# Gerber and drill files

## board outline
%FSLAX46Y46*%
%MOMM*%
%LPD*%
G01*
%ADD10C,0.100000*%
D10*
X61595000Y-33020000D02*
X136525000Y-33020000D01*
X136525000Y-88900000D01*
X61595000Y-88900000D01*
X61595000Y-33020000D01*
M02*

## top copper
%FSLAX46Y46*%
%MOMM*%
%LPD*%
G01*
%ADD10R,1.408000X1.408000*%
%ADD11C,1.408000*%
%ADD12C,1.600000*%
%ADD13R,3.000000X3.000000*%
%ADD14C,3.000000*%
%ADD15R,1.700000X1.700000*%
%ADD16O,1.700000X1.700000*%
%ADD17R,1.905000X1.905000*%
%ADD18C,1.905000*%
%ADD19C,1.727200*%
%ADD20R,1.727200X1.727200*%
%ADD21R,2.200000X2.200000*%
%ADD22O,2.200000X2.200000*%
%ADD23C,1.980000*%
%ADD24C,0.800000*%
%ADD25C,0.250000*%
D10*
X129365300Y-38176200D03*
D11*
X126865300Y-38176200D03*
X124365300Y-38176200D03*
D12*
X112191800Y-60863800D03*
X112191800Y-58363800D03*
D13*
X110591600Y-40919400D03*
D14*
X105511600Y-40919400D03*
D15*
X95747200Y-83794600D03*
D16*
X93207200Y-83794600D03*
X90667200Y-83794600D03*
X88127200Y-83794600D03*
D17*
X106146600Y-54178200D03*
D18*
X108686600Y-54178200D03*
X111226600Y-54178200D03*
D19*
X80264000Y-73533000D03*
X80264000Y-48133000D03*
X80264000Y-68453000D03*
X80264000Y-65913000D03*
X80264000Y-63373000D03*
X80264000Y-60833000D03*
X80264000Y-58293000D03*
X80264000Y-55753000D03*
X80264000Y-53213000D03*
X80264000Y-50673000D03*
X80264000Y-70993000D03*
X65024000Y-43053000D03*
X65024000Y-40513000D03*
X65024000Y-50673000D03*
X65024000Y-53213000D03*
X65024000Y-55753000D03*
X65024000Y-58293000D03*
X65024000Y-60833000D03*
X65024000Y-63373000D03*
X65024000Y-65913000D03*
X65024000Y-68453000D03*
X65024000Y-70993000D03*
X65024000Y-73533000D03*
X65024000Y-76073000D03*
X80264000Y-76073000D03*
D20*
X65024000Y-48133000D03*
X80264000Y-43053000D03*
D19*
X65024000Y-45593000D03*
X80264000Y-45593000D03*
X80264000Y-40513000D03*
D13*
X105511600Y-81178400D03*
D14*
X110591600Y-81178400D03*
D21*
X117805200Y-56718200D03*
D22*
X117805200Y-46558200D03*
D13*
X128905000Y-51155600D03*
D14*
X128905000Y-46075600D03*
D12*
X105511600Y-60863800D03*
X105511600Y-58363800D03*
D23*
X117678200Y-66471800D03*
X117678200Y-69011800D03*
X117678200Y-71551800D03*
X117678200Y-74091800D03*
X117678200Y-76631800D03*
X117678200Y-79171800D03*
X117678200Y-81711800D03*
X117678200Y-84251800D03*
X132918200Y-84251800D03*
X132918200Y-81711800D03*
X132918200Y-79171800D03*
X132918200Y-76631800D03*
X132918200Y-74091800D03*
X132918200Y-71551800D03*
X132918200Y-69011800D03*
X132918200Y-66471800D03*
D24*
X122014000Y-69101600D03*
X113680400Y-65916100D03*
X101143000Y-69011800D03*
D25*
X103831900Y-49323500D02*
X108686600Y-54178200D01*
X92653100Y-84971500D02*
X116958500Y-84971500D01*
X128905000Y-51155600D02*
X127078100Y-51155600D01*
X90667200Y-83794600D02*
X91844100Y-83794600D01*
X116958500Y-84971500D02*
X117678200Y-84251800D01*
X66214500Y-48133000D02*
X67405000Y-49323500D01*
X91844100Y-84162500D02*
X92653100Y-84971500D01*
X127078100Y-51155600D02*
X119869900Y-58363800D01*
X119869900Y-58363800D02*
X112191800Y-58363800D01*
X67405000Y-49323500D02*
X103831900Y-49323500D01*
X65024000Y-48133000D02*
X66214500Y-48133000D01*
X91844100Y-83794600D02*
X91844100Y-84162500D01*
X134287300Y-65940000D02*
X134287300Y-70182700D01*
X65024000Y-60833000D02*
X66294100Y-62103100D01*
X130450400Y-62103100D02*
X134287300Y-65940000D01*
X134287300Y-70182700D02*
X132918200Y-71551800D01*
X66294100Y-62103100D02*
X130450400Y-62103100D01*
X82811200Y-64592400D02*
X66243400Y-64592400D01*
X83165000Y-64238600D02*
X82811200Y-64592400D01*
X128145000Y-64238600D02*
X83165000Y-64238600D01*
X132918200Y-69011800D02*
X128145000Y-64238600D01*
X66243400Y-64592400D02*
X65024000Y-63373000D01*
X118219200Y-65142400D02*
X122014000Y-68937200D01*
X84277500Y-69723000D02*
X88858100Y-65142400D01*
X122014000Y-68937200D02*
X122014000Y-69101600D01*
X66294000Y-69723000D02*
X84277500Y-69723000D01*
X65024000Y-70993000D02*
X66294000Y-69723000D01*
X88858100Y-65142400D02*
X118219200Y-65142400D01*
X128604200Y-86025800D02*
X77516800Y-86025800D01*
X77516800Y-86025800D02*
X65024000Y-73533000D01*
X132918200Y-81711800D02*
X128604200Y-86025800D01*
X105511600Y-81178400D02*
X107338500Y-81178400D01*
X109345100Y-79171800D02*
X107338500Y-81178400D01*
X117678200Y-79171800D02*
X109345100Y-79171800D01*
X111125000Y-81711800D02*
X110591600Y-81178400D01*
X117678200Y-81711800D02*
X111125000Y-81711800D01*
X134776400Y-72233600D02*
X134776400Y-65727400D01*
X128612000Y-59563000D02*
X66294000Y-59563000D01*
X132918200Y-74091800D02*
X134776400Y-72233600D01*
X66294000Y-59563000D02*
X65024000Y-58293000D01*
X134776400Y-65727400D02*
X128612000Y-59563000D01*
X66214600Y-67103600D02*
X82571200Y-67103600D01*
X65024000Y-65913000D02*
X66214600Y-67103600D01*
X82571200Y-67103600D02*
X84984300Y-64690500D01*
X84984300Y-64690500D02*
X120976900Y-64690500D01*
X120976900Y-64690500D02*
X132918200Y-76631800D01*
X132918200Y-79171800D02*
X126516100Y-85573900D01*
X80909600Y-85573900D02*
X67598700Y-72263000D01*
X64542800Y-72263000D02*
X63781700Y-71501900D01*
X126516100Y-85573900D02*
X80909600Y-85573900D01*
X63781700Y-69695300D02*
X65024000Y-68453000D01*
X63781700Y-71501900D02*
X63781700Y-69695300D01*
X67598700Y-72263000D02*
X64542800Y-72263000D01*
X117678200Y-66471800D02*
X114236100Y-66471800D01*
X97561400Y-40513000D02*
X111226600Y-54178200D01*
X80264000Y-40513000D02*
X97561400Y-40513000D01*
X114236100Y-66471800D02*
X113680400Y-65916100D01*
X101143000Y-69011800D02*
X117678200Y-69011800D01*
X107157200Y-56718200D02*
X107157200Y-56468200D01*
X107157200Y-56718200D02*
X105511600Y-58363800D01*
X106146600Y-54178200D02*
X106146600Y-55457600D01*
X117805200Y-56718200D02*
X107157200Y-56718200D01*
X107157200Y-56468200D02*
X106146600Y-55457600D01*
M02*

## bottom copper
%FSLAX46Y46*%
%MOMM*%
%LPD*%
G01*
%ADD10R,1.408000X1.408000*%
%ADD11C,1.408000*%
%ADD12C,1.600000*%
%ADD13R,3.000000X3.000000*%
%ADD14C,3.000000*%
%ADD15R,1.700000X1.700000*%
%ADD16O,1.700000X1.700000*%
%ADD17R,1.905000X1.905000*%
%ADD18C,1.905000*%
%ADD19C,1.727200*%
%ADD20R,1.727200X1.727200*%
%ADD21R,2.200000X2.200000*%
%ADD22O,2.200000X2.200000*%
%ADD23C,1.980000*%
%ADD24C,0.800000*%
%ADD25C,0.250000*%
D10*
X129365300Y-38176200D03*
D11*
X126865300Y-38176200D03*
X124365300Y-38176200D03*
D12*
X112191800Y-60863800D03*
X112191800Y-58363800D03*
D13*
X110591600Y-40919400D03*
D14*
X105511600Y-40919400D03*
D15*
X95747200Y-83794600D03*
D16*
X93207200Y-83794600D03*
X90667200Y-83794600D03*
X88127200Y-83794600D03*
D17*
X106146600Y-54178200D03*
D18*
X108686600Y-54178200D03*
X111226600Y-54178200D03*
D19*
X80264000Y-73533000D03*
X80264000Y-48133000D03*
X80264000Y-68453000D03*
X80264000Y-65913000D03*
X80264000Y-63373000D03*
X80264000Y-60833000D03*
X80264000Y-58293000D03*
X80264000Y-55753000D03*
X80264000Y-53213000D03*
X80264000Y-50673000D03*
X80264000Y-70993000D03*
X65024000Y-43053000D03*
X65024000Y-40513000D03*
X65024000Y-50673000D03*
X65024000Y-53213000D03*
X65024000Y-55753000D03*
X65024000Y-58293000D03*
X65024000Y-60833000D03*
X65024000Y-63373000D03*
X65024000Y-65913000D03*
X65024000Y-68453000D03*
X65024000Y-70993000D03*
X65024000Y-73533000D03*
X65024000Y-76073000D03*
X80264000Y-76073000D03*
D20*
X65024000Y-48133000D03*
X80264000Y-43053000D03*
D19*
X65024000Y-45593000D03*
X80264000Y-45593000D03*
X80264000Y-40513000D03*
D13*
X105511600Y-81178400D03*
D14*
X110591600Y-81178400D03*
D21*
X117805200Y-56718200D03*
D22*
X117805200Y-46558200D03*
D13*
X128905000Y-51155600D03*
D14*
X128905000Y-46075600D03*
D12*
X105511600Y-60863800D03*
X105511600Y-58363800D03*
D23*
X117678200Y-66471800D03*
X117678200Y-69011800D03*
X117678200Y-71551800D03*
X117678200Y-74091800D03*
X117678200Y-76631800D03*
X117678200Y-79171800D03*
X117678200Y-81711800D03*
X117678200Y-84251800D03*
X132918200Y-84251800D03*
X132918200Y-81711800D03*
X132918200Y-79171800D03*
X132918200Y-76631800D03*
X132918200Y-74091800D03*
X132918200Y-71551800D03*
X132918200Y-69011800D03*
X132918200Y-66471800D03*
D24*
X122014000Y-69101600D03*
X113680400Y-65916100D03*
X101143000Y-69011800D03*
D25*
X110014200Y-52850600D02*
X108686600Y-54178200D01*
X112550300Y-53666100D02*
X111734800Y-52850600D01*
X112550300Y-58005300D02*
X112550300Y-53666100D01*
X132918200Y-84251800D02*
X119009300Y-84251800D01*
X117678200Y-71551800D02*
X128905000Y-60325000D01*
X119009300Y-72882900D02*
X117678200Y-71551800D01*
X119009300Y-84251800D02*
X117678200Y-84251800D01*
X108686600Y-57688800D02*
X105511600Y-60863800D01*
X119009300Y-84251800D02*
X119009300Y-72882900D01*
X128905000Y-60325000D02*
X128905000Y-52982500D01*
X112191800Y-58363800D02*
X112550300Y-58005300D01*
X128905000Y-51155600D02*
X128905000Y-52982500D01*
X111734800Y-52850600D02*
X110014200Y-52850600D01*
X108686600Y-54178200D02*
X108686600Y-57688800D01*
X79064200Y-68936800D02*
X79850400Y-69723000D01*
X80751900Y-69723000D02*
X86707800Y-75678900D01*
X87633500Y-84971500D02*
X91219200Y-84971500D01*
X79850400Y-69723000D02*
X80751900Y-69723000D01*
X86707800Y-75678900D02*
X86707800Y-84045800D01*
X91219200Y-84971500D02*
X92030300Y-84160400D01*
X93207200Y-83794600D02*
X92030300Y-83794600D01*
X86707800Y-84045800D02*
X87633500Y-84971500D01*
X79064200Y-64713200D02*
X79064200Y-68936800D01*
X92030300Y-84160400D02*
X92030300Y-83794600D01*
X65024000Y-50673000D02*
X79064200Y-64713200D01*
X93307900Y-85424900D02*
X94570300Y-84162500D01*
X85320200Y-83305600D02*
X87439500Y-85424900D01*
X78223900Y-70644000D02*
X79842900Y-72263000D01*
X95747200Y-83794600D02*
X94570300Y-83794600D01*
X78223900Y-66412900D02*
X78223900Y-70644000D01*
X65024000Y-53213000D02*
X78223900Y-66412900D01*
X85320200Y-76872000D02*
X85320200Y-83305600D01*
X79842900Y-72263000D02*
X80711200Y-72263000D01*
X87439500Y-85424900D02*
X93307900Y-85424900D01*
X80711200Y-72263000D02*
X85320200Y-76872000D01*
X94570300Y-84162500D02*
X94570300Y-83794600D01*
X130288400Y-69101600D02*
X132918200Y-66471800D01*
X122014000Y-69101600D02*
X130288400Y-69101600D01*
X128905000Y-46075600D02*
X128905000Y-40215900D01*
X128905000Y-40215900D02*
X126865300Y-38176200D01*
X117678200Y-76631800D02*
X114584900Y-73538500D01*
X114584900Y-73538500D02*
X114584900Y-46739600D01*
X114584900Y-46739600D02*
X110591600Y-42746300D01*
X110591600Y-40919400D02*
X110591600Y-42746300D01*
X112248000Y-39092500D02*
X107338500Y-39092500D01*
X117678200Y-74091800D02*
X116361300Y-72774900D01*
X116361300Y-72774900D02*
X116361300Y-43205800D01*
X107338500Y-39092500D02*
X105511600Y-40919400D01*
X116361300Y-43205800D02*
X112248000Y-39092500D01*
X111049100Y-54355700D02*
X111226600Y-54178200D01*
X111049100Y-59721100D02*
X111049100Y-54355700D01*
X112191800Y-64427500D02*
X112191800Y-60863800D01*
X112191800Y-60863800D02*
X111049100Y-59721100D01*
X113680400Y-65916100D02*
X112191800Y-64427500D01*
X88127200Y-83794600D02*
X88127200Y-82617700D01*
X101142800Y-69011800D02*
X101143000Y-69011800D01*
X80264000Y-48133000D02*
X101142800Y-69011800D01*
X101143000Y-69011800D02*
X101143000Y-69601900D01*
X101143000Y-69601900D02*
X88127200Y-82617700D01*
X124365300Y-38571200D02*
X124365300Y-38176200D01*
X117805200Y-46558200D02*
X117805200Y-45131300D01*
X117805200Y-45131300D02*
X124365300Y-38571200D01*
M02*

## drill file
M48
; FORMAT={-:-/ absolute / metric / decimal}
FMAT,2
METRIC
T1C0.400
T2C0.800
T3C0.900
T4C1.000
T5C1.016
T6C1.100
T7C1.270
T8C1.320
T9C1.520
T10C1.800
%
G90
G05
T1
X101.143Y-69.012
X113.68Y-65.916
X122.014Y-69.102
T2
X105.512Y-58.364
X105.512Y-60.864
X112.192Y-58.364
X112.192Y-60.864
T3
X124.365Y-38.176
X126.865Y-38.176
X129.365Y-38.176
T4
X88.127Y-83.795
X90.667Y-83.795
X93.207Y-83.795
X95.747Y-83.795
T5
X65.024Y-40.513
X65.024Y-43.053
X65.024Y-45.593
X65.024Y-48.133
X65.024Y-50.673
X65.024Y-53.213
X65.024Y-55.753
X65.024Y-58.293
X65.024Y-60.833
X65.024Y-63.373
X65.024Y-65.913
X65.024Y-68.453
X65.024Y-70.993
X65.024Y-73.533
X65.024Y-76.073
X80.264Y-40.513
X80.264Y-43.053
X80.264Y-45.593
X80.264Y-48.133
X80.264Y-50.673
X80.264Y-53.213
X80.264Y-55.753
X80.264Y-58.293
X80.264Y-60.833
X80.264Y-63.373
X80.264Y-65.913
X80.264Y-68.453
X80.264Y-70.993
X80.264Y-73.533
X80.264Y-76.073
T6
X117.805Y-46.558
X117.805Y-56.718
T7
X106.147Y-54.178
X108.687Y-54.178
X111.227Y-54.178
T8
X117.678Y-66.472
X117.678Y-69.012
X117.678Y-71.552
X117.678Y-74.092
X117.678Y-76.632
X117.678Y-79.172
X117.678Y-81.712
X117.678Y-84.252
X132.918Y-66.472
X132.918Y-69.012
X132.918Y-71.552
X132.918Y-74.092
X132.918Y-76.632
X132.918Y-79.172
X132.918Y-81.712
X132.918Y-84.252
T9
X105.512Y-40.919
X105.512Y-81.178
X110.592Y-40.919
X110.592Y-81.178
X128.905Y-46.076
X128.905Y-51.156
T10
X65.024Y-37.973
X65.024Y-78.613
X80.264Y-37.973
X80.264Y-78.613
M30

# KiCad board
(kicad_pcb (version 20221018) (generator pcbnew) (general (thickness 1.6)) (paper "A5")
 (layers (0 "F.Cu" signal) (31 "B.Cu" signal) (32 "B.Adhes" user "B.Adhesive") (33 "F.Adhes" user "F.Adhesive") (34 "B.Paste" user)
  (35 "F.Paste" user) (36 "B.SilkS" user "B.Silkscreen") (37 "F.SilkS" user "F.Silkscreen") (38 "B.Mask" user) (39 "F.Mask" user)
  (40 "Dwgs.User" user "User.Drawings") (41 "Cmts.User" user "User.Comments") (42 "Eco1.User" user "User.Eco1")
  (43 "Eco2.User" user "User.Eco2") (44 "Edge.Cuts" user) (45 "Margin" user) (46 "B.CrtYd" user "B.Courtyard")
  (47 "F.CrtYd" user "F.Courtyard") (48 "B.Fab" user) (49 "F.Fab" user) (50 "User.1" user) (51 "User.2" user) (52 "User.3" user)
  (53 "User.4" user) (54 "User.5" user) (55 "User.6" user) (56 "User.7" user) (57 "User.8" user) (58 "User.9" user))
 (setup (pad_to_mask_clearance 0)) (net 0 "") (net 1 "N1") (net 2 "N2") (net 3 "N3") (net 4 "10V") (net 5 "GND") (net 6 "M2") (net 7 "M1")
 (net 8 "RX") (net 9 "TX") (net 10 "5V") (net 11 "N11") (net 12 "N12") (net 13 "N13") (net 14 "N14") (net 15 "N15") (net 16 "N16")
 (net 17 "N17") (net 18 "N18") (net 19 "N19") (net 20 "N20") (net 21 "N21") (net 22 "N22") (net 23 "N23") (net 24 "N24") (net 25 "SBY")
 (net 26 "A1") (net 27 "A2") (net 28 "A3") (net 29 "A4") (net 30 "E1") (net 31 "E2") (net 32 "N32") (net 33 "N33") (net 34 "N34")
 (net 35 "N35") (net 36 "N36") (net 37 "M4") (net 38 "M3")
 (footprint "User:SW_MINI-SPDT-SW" (layer "F.Cu") (at 126.8653 38.1762 180)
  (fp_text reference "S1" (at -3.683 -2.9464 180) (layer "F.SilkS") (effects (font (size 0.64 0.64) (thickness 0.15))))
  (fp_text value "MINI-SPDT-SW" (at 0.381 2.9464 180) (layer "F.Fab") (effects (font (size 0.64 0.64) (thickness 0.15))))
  (pad "1" thru_hole rect (at -2.5 0 180) (size 1.408 1.408) (drill 0.9) (layers "*.Cu" "*.Mask") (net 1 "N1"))
  (pad "2" thru_hole circle (at 0 0 180) (size 1.408 1.408) (drill 0.9) (layers "*.Cu" "*.Mask") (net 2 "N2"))
  (pad "3" thru_hole circle (at 2.5 0 180) (size 1.408 1.408) (drill 0.9) (layers "*.Cu" "*.Mask") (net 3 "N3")))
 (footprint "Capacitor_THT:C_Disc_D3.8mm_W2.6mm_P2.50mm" (layer "F.Cu") (at 112.1918 60.8638 90)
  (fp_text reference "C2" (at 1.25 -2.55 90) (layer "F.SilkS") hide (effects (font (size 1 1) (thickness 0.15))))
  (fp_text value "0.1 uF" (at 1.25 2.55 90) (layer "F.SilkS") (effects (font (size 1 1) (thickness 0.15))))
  (pad "1" thru_hole circle (at 0 0 90) (size 1.6 1.6) (drill 0.8) (layers "*.Cu" "*.Mask") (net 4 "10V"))
  (pad "2" thru_hole circle (at 2.5 0 90) (size 1.6 1.6) (drill 0.8) (layers "*.Cu" "*.Mask") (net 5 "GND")))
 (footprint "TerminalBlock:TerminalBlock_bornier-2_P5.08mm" (layer "F.Cu") (at 110.5916 40.9194 180)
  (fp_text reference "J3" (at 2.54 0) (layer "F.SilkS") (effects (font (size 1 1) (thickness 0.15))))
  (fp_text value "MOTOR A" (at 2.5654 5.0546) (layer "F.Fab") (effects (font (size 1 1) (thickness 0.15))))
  (pad "1" thru_hole rect (at 0 0 180) (size 3 3) (drill 1.52) (layers "*.Cu" "*.Mask") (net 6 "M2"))
  (pad "2" thru_hole circle (at 5.08 0 180) (size 3 3) (drill 1.52) (layers "*.Cu" "*.Mask") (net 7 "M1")))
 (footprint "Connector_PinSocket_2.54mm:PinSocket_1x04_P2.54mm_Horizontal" (layer "F.Cu") (at 95.7472 83.7946 -90)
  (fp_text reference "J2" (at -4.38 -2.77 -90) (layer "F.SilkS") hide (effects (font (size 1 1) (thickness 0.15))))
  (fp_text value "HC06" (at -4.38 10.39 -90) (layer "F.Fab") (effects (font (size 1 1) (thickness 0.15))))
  (pad "1" thru_hole rect (at 0 0 270) (size 1.7 1.7) (drill 1) (layers "*.Cu" "*.Mask") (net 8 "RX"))
  (pad "2" thru_hole oval (at 0 2.54 270) (size 1.7 1.7) (drill 1) (layers "*.Cu" "*.Mask") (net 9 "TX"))
  (pad "3" thru_hole oval (at 0 5.08 270) (size 1.7 1.7) (drill 1) (layers "*.Cu" "*.Mask") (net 5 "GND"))
  (pad "4" thru_hole oval (at 0 7.62 270) (size 1.7 1.7) (drill 1) (layers "*.Cu" "*.Mask") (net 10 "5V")))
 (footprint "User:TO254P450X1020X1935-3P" (layer "F.Cu") (at 111.2266 53.086)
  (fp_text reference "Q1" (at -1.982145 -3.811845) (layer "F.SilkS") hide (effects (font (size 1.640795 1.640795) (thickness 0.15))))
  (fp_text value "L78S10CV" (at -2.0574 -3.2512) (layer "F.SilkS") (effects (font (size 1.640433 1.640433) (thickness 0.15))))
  (pad "1" thru_hole rect (at -5.08 1.0922) (size 1.905 1.905) (drill 1.27) (layers "*.Cu" "*.Mask") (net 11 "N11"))
  (pad "2" thru_hole circle (at -2.54 1.0922) (size 1.905 1.905) (drill 1.27) (layers "*.Cu" "*.Mask") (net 5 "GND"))
  (pad "3" thru_hole circle (at 0 1.0922) (size 1.905 1.905) (drill 1.27) (layers "*.Cu" "*.Mask") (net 4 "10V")))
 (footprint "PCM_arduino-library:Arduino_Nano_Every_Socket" (layer "F.Cu") (at 72.644 79.883)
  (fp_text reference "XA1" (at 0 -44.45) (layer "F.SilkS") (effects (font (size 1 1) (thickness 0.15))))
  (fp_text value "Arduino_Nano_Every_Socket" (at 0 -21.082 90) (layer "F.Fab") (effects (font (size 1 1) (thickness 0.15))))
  (pad "" np_thru_hole circle (at -7.62 -41.91) (size 1.8 1.8) (drill 1.8) (layers "F&B.Cu" "*.Mask"))
  (pad "" np_thru_hole circle (at -7.62 -1.27) (size 1.8 1.8) (drill 1.8) (layers "F&B.Cu" "*.Mask"))
  (pad "" np_thru_hole circle (at 7.62 -41.91) (size 1.8 1.8) (drill 1.8) (layers "F&B.Cu" "*.Mask"))
  (pad "" np_thru_hole circle (at 7.62 -1.27) (size 1.8 1.8) (drill 1.8) (layers "F&B.Cu" "*.Mask"))
  (pad "3V3" thru_hole circle (at 7.62 -6.35) (size 1.7272 1.7272) (drill 1.016) (layers "*.Cu" "*.Mask") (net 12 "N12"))
  (pad "5V" thru_hole circle (at 7.62 -31.75) (size 1.7272 1.7272) (drill 1.016) (layers "*.Cu" "*.Mask") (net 10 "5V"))
  (pad "A0" thru_hole circle (at 7.62 -11.43) (size 1.7272 1.7272) (drill 1.016) (layers "*.Cu" "*.Mask") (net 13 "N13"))
  (pad "A1" thru_hole circle (at 7.62 -13.97) (size 1.7272 1.7272) (drill 1.016) (layers "*.Cu" "*.Mask") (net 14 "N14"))
  (pad "A2" thru_hole circle (at 7.62 -16.51) (size 1.7272 1.7272) (drill 1.016) (layers "*.Cu" "*.Mask") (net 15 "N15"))
  (pad "A3" thru_hole circle (at 7.62 -19.05) (size 1.7272 1.7272) (drill 1.016) (layers "*.Cu" "*.Mask") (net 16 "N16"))
  (pad "A4" thru_hole circle (at 7.62 -21.59) (size 1.7272 1.7272) (drill 1.016) (layers "*.Cu" "*.Mask") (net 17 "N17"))
  (pad "A5" thru_hole circle (at 7.62 -24.13) (size 1.7272 1.7272) (drill 1.016) (layers "*.Cu" "*.Mask") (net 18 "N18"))
  (pad "A6" thru_hole circle (at 7.62 -26.67) (size 1.7272 1.7272) (drill 1.016) (layers "*.Cu" "*.Mask") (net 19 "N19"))
  (pad "A7" thru_hole circle (at 7.62 -29.21) (size 1.7272 1.7272) (drill 1.016) (layers "*.Cu" "*.Mask") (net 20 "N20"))
  (pad "AREF" thru_hole circle (at 7.62 -8.89) (size 1.7272 1.7272) (drill 1.016) (layers "*.Cu" "*.Mask") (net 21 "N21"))
  (pad "D0" thru_hole circle (at -7.62 -36.83) (size 1.7272 1.7272) (drill 1.016) (layers "*.Cu" "*.Mask") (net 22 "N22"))
  (pad "D1" thru_hole circle (at -7.62 -39.37) (size 1.7272 1.7272) (drill 1.016) (layers "*.Cu" "*.Mask") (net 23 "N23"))
  (pad "D2" thru_hole circle (at -7.62 -29.21) (size 1.7272 1.7272) (drill 1.016) (layers "*.Cu" "*.Mask") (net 9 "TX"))
  (pad "D3" thru_hole circle (at -7.62 -26.67) (size 1.7272 1.7272) (drill 1.016) (layers "*.Cu" "*.Mask") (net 8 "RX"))
  (pad "D4" thru_hole circle (at -7.62 -24.13) (size 1.7272 1.7272) (drill 1.016) (layers "*.Cu" "*.Mask") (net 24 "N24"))
  (pad "D5" thru_hole circle (at -7.62 -21.59) (size 1.7272 1.7272) (drill 1.016) (layers "*.Cu" "*.Mask") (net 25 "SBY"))
  (pad "D6" thru_hole circle (at -7.62 -19.05) (size 1.7272 1.7272) (drill 1.016) (layers "*.Cu" "*.Mask") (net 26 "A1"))
  (pad "D7" thru_hole circle (at -7.62 -16.51) (size 1.7272 1.7272) (drill 1.016) (layers "*.Cu" "*.Mask") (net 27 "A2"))
  (pad "D8" thru_hole circle (at -7.62 -13.97) (size 1.7272 1.7272) (drill 1.016) (layers "*.Cu" "*.Mask") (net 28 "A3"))
  (pad "D9" thru_hole circle (at -7.62 -11.43) (size 1.7272 1.7272) (drill 1.016) (layers "*.Cu" "*.Mask") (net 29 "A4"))
  (pad "D10" thru_hole circle (at -7.62 -8.89) (size 1.7272 1.7272) (drill 1.016) (layers "*.Cu" "*.Mask") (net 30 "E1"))
  (pad "D11" thru_hole circle (at -7.62 -6.35) (size 1.7272 1.7272) (drill 1.016) (layers "*.Cu" "*.Mask") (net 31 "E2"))
  (pad "D12" thru_hole circle (at -7.62 -3.81) (size 1.7272 1.7272) (drill 1.016) (layers "*.Cu" "*.Mask") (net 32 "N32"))
  (pad "D13" thru_hole circle (at 7.62 -3.81) (size 1.7272 1.7272) (drill 1.016) (layers "*.Cu" "*.Mask") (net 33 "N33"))
  (pad "GND1" thru_hole rect (at -7.62 -31.75) (size 1.7272 1.7272) (drill 1.016) (layers "*.Cu" "*.Mask") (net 5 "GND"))
  (pad "GND2" thru_hole rect (at 7.62 -36.83) (size 1.7272 1.7272) (drill 1.016) (layers "*.Cu" "*.Mask") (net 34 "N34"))
  (pad "RST1" thru_hole circle (at -7.62 -34.29) (size 1.7272 1.7272) (drill 1.016) (layers "*.Cu" "*.Mask") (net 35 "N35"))
  (pad "RST2" thru_hole circle (at 7.62 -34.29) (size 1.7272 1.7272) (drill 1.016) (layers "*.Cu" "*.Mask") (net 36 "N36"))
  (pad "VIN" thru_hole circle (at 7.62 -39.37) (size 1.7272 1.7272) (drill 1.016) (layers "*.Cu" "*.Mask") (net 4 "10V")))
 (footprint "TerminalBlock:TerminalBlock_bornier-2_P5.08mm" (layer "F.Cu") (at 105.5116 81.1784)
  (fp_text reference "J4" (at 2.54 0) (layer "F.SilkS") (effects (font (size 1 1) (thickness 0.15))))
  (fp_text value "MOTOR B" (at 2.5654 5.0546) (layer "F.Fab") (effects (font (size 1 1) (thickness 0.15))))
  (pad "1" thru_hole rect (at 0 0) (size 3 3) (drill 1.52) (layers "*.Cu" "*.Mask") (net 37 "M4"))
  (pad "2" thru_hole circle (at 5.08 0) (size 3 3) (drill 1.52) (layers "*.Cu" "*.Mask") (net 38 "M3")))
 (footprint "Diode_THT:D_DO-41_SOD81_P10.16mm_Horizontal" (layer "F.Cu") (at 117.8052 56.7182 90)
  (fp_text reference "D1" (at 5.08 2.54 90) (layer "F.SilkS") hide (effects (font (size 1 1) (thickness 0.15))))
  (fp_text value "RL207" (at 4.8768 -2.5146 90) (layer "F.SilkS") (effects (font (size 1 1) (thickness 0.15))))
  (pad "1" thru_hole rect (at 0 0 90) (size 2.2 2.2) (drill 1.1) (layers "*.Cu" "*.Mask") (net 11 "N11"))
  (pad "2" thru_hole oval (at 10.16 0 90) (size 2.2 2.2) (drill 1.1) (layers "*.Cu" "*.Mask") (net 3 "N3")))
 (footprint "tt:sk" (layer "F.Cu") (at 128.111013 59.633485)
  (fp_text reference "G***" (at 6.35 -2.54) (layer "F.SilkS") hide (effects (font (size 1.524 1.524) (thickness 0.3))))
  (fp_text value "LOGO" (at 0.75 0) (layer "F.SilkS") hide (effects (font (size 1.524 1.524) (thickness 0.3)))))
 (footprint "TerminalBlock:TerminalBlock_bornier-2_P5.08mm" (layer "F.Cu") (at 128.905 51.1556 90)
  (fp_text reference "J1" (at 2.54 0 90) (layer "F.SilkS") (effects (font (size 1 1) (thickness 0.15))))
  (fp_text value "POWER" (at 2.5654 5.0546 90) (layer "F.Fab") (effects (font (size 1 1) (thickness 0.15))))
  (pad "1" thru_hole rect (at 0 0 90) (size 3 3) (drill 1.52) (layers "*.Cu" "*.Mask") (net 5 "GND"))
  (pad "2" thru_hole circle (at 5.08 0 90) (size 3 3) (drill 1.52) (layers "*.Cu" "*.Mask") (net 2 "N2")))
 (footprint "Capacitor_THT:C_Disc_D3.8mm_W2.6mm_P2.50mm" (layer "F.Cu") (at 105.5116 60.8638 90)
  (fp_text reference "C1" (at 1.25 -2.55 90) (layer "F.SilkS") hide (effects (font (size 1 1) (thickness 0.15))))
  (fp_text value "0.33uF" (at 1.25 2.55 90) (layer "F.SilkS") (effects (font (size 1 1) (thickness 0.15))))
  (pad "1" thru_hole circle (at 0 0 90) (size 1.6 1.6) (drill 0.8) (layers "*.Cu" "*.Mask") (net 5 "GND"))
  (pad "2" thru_hole circle (at 2.5 0 90) (size 1.6 1.6) (drill 0.8) (layers "*.Cu" "*.Mask") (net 11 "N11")))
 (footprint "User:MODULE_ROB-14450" (layer "F.Cu") (at 125.2982 75.3618)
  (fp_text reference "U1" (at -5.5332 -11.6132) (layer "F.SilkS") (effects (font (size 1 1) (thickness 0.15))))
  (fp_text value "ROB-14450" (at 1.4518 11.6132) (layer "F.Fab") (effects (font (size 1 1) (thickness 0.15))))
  (pad "1" thru_hole circle (at -7.62 -8.89) (size 1.98 1.98) (drill 1.32) (layers "*.Cu" "*.Mask") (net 4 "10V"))
  (pad "2" thru_hole circle (at -7.62 -6.35) (size 1.98 1.98) (drill 1.32) (layers "*.Cu" "*.Mask") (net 10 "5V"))
  (pad "3" thru_hole circle (at -7.62 -3.81) (size 1.98 1.98) (drill 1.32) (layers "*.Cu" "*.Mask") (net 5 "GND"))
  (pad "4" thru_hole circle (at -7.62 -1.27) (size 1.98 1.98) (drill 1.32) (layers "*.Cu" "*.Mask") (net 7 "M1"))
  (pad "5" thru_hole circle (at -7.62 1.27) (size 1.98 1.98) (drill 1.32) (layers "*.Cu" "*.Mask") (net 6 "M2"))
  (pad "6" thru_hole circle (at -7.62 3.81) (size 1.98 1.98) (drill 1.32) (layers "*.Cu" "*.Mask") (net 37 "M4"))
  (pad "7" thru_hole circle (at -7.62 6.35) (size 1.98 1.98) (drill 1.32) (layers "*.Cu" "*.Mask") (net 38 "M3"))
  (pad "8" thru_hole circle (at -7.62 8.89) (size 1.98 1.98) (drill 1.32) (layers "*.Cu" "*.Mask") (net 5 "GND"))
  (pad "9" thru_hole circle (at 7.62 8.89) (size 1.98 1.98) (drill 1.32) (layers "*.Cu" "*.Mask") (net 5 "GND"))
  (pad "10" thru_hole circle (at 7.62 6.35) (size 1.98 1.98) (drill 1.32) (layers "*.Cu" "*.Mask") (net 31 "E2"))
  (pad "11" thru_hole circle (at 7.62 3.81) (size 1.98 1.98) (drill 1.32) (layers "*.Cu" "*.Mask") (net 29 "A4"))
  (pad "12" thru_hole circle (at 7.62 1.27) (size 1.98 1.98) (drill 1.32) (layers "*.Cu" "*.Mask") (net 28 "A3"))
  (pad "13" thru_hole circle (at 7.62 -1.27) (size 1.98 1.98) (drill 1.32) (layers "*.Cu" "*.Mask") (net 25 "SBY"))
  (pad "14" thru_hole circle (at 7.62 -3.81) (size 1.98 1.98) (drill 1.32) (layers "*.Cu" "*.Mask") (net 26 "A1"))
  (pad "15" thru_hole circle (at 7.62 -6.35) (size 1.98 1.98) (drill 1.32) (layers "*.Cu" "*.Mask") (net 27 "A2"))
  (pad "16" thru_hole circle (at 7.62 -8.89) (size 1.98 1.98) (drill 1.32) (layers "*.Cu" "*.Mask") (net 30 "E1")))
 (gr_rect (start 61.595 33.02) (end 136.525 88.9) (stroke (width 0.1) (type solid)) (fill none) (layer "Edge.Cuts"))
 (segment (start 103.8319 49.3235) (end 108.6866 54.1782) (width 0.25) (layer "F.Cu") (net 5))
 (segment (start 92.6531 84.9715) (end 116.9585 84.9715) (width 0.25) (layer "F.Cu") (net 5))
 (segment (start 128.905 51.1556) (end 127.0781 51.1556) (width 0.25) (layer "F.Cu") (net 5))
 (segment (start 90.6672 83.7946) (end 91.8441 83.7946) (width 0.25) (layer "F.Cu") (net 5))
 (segment (start 116.9585 84.9715) (end 117.6782 84.2518) (width 0.25) (layer "F.Cu") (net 5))
 (segment (start 66.2145 48.133) (end 67.405 49.3235) (width 0.25) (layer "F.Cu") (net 5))
 (segment (start 91.8441 84.1625) (end 92.6531 84.9715) (width 0.25) (layer "F.Cu") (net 5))
 (segment (start 127.0781 51.1556) (end 119.8699 58.3638) (width 0.25) (layer "F.Cu") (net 5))
 (segment (start 119.8699 58.3638) (end 112.1918 58.3638) (width 0.25) (layer "F.Cu") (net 5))
 (segment (start 67.405 49.3235) (end 103.8319 49.3235) (width 0.25) (layer "F.Cu") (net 5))
 (segment (start 65.024 48.133) (end 66.2145 48.133) (width 0.25) (layer "F.Cu") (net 5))
 (segment (start 91.8441 83.7946) (end 91.8441 84.1625) (width 0.25) (layer "F.Cu") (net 5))
 (segment (start 110.0142 52.8506) (end 108.6866 54.1782) (width 0.25) (layer "B.Cu") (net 5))
 (segment (start 112.5503 53.6661) (end 111.7348 52.8506) (width 0.25) (layer "B.Cu") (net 5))
 (segment (start 112.5503 58.0053) (end 112.5503 53.6661) (width 0.25) (layer "B.Cu") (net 5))
 (segment (start 132.9182 84.2518) (end 119.0093 84.2518) (width 0.25) (layer "B.Cu") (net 5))
 (segment (start 117.6782 71.5518) (end 128.905 60.325) (width 0.25) (layer "B.Cu") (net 5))
 (segment (start 119.0093 72.8829) (end 117.6782 71.5518) (width 0.25) (layer "B.Cu") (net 5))
 (segment (start 119.0093 84.2518) (end 117.6782 84.2518) (width 0.25) (layer "B.Cu") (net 5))
 (segment (start 108.6866 57.6888) (end 105.5116 60.8638) (width 0.25) (layer "B.Cu") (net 5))
 (segment (start 119.0093 84.2518) (end 119.0093 72.8829) (width 0.25) (layer "B.Cu") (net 5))
 (segment (start 128.905 60.325) (end 128.905 52.9825) (width 0.25) (layer "B.Cu") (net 5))
 (segment (start 112.1918 58.3638) (end 112.5503 58.0053) (width 0.25) (layer "B.Cu") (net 5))
 (segment (start 128.905 51.1556) (end 128.905 52.9825) (width 0.25) (layer "B.Cu") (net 5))
 (segment (start 111.7348 52.8506) (end 110.0142 52.8506) (width 0.25) (layer "B.Cu") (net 5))
 (segment (start 108.6866 54.1782) (end 108.6866 57.6888) (width 0.25) (layer "B.Cu") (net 5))
 (segment (start 79.0642 68.9368) (end 79.8504 69.723) (width 0.25) (layer "B.Cu") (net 9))
 (segment (start 80.7519 69.723) (end 86.7078 75.6789) (width 0.25) (layer "B.Cu") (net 9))
 (segment (start 87.6335 84.9715) (end 91.2192 84.9715) (width 0.25) (layer "B.Cu") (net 9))
 (segment (start 79.8504 69.723) (end 80.7519 69.723) (width 0.25) (layer "B.Cu") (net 9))
 (segment (start 86.7078 75.6789) (end 86.7078 84.0458) (width 0.25) (layer "B.Cu") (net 9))
 (segment (start 91.2192 84.9715) (end 92.0303 84.1604) (width 0.25) (layer "B.Cu") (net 9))
 (segment (start 93.2072 83.7946) (end 92.0303 83.7946) (width 0.25) (layer "B.Cu") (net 9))
 (segment (start 86.7078 84.0458) (end 87.6335 84.9715) (width 0.25) (layer "B.Cu") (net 9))
 (segment (start 79.0642 64.7132) (end 79.0642 68.9368) (width 0.25) (layer "B.Cu") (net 9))
 (segment (start 92.0303 84.1604) (end 92.0303 83.7946) (width 0.25) (layer "B.Cu") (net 9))
 (segment (start 65.024 50.673) (end 79.0642 64.7132) (width 0.25) (layer "B.Cu") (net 9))
 (segment (start 93.3079 85.4249) (end 94.5703 84.1625) (width 0.25) (layer "B.Cu") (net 8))
 (segment (start 85.3202 83.3056) (end 87.4395 85.4249) (width 0.25) (layer "B.Cu") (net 8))
 (segment (start 78.2239 70.644) (end 79.8429 72.263) (width 0.25) (layer "B.Cu") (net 8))
 (segment (start 95.7472 83.7946) (end 94.5703 83.7946) (width 0.25) (layer "B.Cu") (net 8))
 (segment (start 78.2239 66.4129) (end 78.2239 70.644) (width 0.25) (layer "B.Cu") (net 8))
 (segment (start 65.024 53.213) (end 78.2239 66.4129) (width 0.25) (layer "B.Cu") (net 8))
 (segment (start 85.3202 76.872) (end 85.3202 83.3056) (width 0.25) (layer "B.Cu") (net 8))
 (segment (start 79.8429 72.263) (end 80.7112 72.263) (width 0.25) (layer "B.Cu") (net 8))
 (segment (start 87.4395 85.4249) (end 93.3079 85.4249) (width 0.25) (layer "B.Cu") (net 8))
 (segment (start 80.7112 72.263) (end 85.3202 76.872) (width 0.25) (layer "B.Cu") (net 8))
 (segment (start 94.5703 84.1625) (end 94.5703 83.7946) (width 0.25) (layer "B.Cu") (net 8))
 (segment (start 134.2873 65.94) (end 134.2873 70.1827) (width 0.25) (layer "F.Cu") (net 26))
 (segment (start 65.024 60.833) (end 66.2941 62.1031) (width 0.25) (layer "F.Cu") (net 26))
 (segment (start 130.4504 62.1031) (end 134.2873 65.94) (width 0.25) (layer "F.Cu") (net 26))
 (segment (start 134.2873 70.1827) (end 132.9182 71.5518) (width 0.25) (layer "F.Cu") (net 26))
 (segment (start 66.2941 62.1031) (end 130.4504 62.1031) (width 0.25) (layer "F.Cu") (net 26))
 (segment (start 82.8112 64.5924) (end 66.2434 64.5924) (width 0.25) (layer "F.Cu") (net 27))
 (segment (start 83.165 64.2386) (end 82.8112 64.5924) (width 0.25) (layer "F.Cu") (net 27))
 (segment (start 128.145 64.2386) (end 83.165 64.2386) (width 0.25) (layer "F.Cu") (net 27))
 (segment (start 132.9182 69.0118) (end 128.145 64.2386) (width 0.25) (layer "F.Cu") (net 27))
 (segment (start 66.2434 64.5924) (end 65.024 63.373) (width 0.25) (layer "F.Cu") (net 27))
 (segment (start 118.2192 65.1424) (end 122.014 68.9372) (width 0.25) (layer "F.Cu") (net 30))
 (segment (start 84.2775 69.723) (end 88.8581 65.1424) (width 0.25) (layer "F.Cu") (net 30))
 (segment (start 122.014 68.9372) (end 122.014 69.1016) (width 0.25) (layer "F.Cu") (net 30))
 (segment (start 66.294 69.723) (end 84.2775 69.723) (width 0.25) (layer "F.Cu") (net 30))
 (segment (start 65.024 70.993) (end 66.294 69.723) (width 0.25) (layer "F.Cu") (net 30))
 (segment (start 88.8581 65.1424) (end 118.2192 65.1424) (width 0.25) (layer "F.Cu") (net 30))
 (via (at 122.014 69.1016) (size 0.8) (drill 0.4) (layers "F.Cu" "B.Cu") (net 30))
 (segment (start 130.2884 69.1016) (end 132.9182 66.4718) (width 0.25) (layer "B.Cu") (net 30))
 (segment (start 122.014 69.1016) (end 130.2884 69.1016) (width 0.25) (layer "B.Cu") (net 30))
 (segment (start 128.6042 86.0258) (end 77.5168 86.0258) (width 0.25) (layer "F.Cu") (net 31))
 (segment (start 77.5168 86.0258) (end 65.024 73.533) (width 0.25) (layer "F.Cu") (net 31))
 (segment (start 132.9182 81.7118) (end 128.6042 86.0258) (width 0.25) (layer "F.Cu") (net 31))
 (segment (start 128.905 46.0756) (end 128.905 40.2159) (width 0.25) (layer "B.Cu") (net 2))
 (segment (start 128.905 40.2159) (end 126.8653 38.1762) (width 0.25) (layer "B.Cu") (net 2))
 (segment (start 117.6782 76.6318) (end 114.5849 73.5385) (width 0.25) (layer "B.Cu") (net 6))
 (segment (start 114.5849 73.5385) (end 114.5849 46.7396) (width 0.25) (layer "B.Cu") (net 6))
 (segment (start 114.5849 46.7396) (end 110.5916 42.7463) (width 0.25) (layer "B.Cu") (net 6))
 (segment (start 110.5916 40.9194) (end 110.5916 42.7463) (width 0.25) (layer "B.Cu") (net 6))
 (segment (start 112.248 39.0925) (end 107.3385 39.0925) (width 0.25) (layer "B.Cu") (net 7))
 (segment (start 117.6782 74.0918) (end 116.3613 72.7749) (width 0.25) (layer "B.Cu") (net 7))
 (segment (start 116.3613 72.7749) (end 116.3613 43.2058) (width 0.25) (layer "B.Cu") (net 7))
 (segment (start 107.3385 39.0925) (end 105.5116 40.9194) (width 0.25) (layer "B.Cu") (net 7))
 (segment (start 116.3613 43.2058) (end 112.248 39.0925) (width 0.25) (layer "B.Cu") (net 7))
 (segment (start 105.5116 81.1784) (end 107.3385 81.1784) (width 0.25) (layer "F.Cu") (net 37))
 (segment (start 109.3451 79.1718) (end 107.3385 81.1784) (width 0.25) (layer "F.Cu") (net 37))
 (segment (start 117.6782 79.1718) (end 109.3451 79.1718) (width 0.25) (layer "F.Cu") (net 37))
 (segment (start 111.125 81.7118) (end 110.5916 81.1784) (width 0.25) (layer "F.Cu") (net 38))
 (segment (start 117.6782 81.7118) (end 111.125 81.7118) (width 0.25) (layer "F.Cu") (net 38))
 (segment (start 134.7764 72.2336) (end 134.7764 65.7274) (width 0.25) (layer "F.Cu") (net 25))
 (segment (start 128.612 59.563) (end 66.294 59.563) (width 0.25) (layer "F.Cu") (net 25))
 (segment (start 132.9182 74.0918) (end 134.7764 72.2336) (width 0.25) (layer "F.Cu") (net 25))
 (segment (start 66.294 59.563) (end 65.024 58.293) (width 0.25) (layer "F.Cu") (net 25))
 (segment (start 134.7764 65.7274) (end 128.612 59.563) (width 0.25) (layer "F.Cu") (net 25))
 (segment (start 66.2146 67.1036) (end 82.5712 67.1036) (width 0.25) (layer "F.Cu") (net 28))
 (segment (start 65.024 65.913) (end 66.2146 67.1036) (width 0.25) (layer "F.Cu") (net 28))
 (segment (start 82.5712 67.1036) (end 84.9843 64.6905) (width 0.25) (layer "F.Cu") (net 28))
 (segment (start 84.9843 64.6905) (end 120.9769 64.6905) (width 0.25) (layer "F.Cu") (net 28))
 (segment (start 120.9769 64.6905) (end 132.9182 76.6318) (width 0.25) (layer "F.Cu") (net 28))
 (segment (start 132.9182 79.1718) (end 126.5161 85.5739) (width 0.25) (layer "F.Cu") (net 29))
 (segment (start 80.9096 85.5739) (end 67.5987 72.263) (width 0.25) (layer "F.Cu") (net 29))
 (segment (start 64.5428 72.263) (end 63.7817 71.5019) (width 0.25) (layer "F.Cu") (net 29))
 (segment (start 126.5161 85.5739) (end 80.9096 85.5739) (width 0.25) (layer "F.Cu") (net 29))
 (segment (start 63.7817 69.6953) (end 65.024 68.453) (width 0.25) (layer "F.Cu") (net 29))
 (segment (start 63.7817 71.5019) (end 63.7817 69.6953) (width 0.25) (layer "F.Cu") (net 29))
 (segment (start 67.5987 72.263) (end 64.5428 72.263) (width 0.25) (layer "F.Cu") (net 29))
 (segment (start 117.6782 66.4718) (end 114.2361 66.4718) (width 0.25) (layer "F.Cu") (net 4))
 (segment (start 97.5614 40.513) (end 111.2266 54.1782) (width 0.25) (layer "F.Cu") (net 4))
 (segment (start 80.264 40.513) (end 97.5614 40.513) (width 0.25) (layer "F.Cu") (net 4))
 (segment (start 114.2361 66.4718) (end 113.6804 65.9161) (width 0.25) (layer "F.Cu") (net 4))
 (via (at 113.6804 65.9161) (size 0.8) (drill 0.4) (layers "F.Cu" "B.Cu") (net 4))
 (segment (start 111.0491 54.3557) (end 111.2266 54.1782) (width 0.25) (layer "B.Cu") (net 4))
 (segment (start 111.0491 59.7211) (end 111.0491 54.3557) (width 0.25) (layer "B.Cu") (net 4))
 (segment (start 112.1918 64.4275) (end 112.1918 60.8638) (width 0.25) (layer "B.Cu") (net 4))
 (segment (start 112.1918 60.8638) (end 111.0491 59.7211) (width 0.25) (layer "B.Cu") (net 4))
 (segment (start 113.6804 65.9161) (end 112.1918 64.4275) (width 0.25) (layer "B.Cu") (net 4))
 (segment (start 101.143 69.0118) (end 117.6782 69.0118) (width 0.25) (layer "F.Cu") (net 10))
 (via (at 101.143 69.0118) (size 0.8) (drill 0.4) (layers "F.Cu" "B.Cu") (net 10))
 (segment (start 88.1272 83.7946) (end 88.1272 82.6177) (width 0.25) (layer "B.Cu") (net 10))
 (segment (start 101.1428 69.0118) (end 101.143 69.0118) (width 0.25) (layer "B.Cu") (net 10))
 (segment (start 80.264 48.133) (end 101.1428 69.0118) (width 0.25) (layer "B.Cu") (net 10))
 (segment (start 101.143 69.0118) (end 101.143 69.6019) (width 0.25) (layer "B.Cu") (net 10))
 (segment (start 101.143 69.6019) (end 88.1272 82.6177) (width 0.25) (layer "B.Cu") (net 10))
 (segment (start 107.1572 56.7182) (end 107.1572 56.4682) (width 0.25) (layer "F.Cu") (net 11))
 (segment (start 107.1572 56.7182) (end 105.5116 58.3638) (width 0.25) (layer "F.Cu") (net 11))
 (segment (start 106.1466 54.1782) (end 106.1466 55.4576) (width 0.25) (layer "F.Cu") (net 11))
 (segment (start 117.8052 56.7182) (end 107.1572 56.7182) (width 0.25) (layer "F.Cu") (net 11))
 (segment (start 107.1572 56.4682) (end 106.1466 55.4576) (width 0.25) (layer "F.Cu") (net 11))
 (segment (start 124.3653 38.5712) (end 124.3653 38.1762) (width 0.25) (layer "B.Cu") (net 3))
 (segment (start 117.8052 46.5582) (end 117.8052 45.1313) (width 0.25) (layer "B.Cu") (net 3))
 (segment (start 117.8052 45.1313) (end 124.3653 38.5712) (width 0.25) (layer "B.Cu") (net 3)))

